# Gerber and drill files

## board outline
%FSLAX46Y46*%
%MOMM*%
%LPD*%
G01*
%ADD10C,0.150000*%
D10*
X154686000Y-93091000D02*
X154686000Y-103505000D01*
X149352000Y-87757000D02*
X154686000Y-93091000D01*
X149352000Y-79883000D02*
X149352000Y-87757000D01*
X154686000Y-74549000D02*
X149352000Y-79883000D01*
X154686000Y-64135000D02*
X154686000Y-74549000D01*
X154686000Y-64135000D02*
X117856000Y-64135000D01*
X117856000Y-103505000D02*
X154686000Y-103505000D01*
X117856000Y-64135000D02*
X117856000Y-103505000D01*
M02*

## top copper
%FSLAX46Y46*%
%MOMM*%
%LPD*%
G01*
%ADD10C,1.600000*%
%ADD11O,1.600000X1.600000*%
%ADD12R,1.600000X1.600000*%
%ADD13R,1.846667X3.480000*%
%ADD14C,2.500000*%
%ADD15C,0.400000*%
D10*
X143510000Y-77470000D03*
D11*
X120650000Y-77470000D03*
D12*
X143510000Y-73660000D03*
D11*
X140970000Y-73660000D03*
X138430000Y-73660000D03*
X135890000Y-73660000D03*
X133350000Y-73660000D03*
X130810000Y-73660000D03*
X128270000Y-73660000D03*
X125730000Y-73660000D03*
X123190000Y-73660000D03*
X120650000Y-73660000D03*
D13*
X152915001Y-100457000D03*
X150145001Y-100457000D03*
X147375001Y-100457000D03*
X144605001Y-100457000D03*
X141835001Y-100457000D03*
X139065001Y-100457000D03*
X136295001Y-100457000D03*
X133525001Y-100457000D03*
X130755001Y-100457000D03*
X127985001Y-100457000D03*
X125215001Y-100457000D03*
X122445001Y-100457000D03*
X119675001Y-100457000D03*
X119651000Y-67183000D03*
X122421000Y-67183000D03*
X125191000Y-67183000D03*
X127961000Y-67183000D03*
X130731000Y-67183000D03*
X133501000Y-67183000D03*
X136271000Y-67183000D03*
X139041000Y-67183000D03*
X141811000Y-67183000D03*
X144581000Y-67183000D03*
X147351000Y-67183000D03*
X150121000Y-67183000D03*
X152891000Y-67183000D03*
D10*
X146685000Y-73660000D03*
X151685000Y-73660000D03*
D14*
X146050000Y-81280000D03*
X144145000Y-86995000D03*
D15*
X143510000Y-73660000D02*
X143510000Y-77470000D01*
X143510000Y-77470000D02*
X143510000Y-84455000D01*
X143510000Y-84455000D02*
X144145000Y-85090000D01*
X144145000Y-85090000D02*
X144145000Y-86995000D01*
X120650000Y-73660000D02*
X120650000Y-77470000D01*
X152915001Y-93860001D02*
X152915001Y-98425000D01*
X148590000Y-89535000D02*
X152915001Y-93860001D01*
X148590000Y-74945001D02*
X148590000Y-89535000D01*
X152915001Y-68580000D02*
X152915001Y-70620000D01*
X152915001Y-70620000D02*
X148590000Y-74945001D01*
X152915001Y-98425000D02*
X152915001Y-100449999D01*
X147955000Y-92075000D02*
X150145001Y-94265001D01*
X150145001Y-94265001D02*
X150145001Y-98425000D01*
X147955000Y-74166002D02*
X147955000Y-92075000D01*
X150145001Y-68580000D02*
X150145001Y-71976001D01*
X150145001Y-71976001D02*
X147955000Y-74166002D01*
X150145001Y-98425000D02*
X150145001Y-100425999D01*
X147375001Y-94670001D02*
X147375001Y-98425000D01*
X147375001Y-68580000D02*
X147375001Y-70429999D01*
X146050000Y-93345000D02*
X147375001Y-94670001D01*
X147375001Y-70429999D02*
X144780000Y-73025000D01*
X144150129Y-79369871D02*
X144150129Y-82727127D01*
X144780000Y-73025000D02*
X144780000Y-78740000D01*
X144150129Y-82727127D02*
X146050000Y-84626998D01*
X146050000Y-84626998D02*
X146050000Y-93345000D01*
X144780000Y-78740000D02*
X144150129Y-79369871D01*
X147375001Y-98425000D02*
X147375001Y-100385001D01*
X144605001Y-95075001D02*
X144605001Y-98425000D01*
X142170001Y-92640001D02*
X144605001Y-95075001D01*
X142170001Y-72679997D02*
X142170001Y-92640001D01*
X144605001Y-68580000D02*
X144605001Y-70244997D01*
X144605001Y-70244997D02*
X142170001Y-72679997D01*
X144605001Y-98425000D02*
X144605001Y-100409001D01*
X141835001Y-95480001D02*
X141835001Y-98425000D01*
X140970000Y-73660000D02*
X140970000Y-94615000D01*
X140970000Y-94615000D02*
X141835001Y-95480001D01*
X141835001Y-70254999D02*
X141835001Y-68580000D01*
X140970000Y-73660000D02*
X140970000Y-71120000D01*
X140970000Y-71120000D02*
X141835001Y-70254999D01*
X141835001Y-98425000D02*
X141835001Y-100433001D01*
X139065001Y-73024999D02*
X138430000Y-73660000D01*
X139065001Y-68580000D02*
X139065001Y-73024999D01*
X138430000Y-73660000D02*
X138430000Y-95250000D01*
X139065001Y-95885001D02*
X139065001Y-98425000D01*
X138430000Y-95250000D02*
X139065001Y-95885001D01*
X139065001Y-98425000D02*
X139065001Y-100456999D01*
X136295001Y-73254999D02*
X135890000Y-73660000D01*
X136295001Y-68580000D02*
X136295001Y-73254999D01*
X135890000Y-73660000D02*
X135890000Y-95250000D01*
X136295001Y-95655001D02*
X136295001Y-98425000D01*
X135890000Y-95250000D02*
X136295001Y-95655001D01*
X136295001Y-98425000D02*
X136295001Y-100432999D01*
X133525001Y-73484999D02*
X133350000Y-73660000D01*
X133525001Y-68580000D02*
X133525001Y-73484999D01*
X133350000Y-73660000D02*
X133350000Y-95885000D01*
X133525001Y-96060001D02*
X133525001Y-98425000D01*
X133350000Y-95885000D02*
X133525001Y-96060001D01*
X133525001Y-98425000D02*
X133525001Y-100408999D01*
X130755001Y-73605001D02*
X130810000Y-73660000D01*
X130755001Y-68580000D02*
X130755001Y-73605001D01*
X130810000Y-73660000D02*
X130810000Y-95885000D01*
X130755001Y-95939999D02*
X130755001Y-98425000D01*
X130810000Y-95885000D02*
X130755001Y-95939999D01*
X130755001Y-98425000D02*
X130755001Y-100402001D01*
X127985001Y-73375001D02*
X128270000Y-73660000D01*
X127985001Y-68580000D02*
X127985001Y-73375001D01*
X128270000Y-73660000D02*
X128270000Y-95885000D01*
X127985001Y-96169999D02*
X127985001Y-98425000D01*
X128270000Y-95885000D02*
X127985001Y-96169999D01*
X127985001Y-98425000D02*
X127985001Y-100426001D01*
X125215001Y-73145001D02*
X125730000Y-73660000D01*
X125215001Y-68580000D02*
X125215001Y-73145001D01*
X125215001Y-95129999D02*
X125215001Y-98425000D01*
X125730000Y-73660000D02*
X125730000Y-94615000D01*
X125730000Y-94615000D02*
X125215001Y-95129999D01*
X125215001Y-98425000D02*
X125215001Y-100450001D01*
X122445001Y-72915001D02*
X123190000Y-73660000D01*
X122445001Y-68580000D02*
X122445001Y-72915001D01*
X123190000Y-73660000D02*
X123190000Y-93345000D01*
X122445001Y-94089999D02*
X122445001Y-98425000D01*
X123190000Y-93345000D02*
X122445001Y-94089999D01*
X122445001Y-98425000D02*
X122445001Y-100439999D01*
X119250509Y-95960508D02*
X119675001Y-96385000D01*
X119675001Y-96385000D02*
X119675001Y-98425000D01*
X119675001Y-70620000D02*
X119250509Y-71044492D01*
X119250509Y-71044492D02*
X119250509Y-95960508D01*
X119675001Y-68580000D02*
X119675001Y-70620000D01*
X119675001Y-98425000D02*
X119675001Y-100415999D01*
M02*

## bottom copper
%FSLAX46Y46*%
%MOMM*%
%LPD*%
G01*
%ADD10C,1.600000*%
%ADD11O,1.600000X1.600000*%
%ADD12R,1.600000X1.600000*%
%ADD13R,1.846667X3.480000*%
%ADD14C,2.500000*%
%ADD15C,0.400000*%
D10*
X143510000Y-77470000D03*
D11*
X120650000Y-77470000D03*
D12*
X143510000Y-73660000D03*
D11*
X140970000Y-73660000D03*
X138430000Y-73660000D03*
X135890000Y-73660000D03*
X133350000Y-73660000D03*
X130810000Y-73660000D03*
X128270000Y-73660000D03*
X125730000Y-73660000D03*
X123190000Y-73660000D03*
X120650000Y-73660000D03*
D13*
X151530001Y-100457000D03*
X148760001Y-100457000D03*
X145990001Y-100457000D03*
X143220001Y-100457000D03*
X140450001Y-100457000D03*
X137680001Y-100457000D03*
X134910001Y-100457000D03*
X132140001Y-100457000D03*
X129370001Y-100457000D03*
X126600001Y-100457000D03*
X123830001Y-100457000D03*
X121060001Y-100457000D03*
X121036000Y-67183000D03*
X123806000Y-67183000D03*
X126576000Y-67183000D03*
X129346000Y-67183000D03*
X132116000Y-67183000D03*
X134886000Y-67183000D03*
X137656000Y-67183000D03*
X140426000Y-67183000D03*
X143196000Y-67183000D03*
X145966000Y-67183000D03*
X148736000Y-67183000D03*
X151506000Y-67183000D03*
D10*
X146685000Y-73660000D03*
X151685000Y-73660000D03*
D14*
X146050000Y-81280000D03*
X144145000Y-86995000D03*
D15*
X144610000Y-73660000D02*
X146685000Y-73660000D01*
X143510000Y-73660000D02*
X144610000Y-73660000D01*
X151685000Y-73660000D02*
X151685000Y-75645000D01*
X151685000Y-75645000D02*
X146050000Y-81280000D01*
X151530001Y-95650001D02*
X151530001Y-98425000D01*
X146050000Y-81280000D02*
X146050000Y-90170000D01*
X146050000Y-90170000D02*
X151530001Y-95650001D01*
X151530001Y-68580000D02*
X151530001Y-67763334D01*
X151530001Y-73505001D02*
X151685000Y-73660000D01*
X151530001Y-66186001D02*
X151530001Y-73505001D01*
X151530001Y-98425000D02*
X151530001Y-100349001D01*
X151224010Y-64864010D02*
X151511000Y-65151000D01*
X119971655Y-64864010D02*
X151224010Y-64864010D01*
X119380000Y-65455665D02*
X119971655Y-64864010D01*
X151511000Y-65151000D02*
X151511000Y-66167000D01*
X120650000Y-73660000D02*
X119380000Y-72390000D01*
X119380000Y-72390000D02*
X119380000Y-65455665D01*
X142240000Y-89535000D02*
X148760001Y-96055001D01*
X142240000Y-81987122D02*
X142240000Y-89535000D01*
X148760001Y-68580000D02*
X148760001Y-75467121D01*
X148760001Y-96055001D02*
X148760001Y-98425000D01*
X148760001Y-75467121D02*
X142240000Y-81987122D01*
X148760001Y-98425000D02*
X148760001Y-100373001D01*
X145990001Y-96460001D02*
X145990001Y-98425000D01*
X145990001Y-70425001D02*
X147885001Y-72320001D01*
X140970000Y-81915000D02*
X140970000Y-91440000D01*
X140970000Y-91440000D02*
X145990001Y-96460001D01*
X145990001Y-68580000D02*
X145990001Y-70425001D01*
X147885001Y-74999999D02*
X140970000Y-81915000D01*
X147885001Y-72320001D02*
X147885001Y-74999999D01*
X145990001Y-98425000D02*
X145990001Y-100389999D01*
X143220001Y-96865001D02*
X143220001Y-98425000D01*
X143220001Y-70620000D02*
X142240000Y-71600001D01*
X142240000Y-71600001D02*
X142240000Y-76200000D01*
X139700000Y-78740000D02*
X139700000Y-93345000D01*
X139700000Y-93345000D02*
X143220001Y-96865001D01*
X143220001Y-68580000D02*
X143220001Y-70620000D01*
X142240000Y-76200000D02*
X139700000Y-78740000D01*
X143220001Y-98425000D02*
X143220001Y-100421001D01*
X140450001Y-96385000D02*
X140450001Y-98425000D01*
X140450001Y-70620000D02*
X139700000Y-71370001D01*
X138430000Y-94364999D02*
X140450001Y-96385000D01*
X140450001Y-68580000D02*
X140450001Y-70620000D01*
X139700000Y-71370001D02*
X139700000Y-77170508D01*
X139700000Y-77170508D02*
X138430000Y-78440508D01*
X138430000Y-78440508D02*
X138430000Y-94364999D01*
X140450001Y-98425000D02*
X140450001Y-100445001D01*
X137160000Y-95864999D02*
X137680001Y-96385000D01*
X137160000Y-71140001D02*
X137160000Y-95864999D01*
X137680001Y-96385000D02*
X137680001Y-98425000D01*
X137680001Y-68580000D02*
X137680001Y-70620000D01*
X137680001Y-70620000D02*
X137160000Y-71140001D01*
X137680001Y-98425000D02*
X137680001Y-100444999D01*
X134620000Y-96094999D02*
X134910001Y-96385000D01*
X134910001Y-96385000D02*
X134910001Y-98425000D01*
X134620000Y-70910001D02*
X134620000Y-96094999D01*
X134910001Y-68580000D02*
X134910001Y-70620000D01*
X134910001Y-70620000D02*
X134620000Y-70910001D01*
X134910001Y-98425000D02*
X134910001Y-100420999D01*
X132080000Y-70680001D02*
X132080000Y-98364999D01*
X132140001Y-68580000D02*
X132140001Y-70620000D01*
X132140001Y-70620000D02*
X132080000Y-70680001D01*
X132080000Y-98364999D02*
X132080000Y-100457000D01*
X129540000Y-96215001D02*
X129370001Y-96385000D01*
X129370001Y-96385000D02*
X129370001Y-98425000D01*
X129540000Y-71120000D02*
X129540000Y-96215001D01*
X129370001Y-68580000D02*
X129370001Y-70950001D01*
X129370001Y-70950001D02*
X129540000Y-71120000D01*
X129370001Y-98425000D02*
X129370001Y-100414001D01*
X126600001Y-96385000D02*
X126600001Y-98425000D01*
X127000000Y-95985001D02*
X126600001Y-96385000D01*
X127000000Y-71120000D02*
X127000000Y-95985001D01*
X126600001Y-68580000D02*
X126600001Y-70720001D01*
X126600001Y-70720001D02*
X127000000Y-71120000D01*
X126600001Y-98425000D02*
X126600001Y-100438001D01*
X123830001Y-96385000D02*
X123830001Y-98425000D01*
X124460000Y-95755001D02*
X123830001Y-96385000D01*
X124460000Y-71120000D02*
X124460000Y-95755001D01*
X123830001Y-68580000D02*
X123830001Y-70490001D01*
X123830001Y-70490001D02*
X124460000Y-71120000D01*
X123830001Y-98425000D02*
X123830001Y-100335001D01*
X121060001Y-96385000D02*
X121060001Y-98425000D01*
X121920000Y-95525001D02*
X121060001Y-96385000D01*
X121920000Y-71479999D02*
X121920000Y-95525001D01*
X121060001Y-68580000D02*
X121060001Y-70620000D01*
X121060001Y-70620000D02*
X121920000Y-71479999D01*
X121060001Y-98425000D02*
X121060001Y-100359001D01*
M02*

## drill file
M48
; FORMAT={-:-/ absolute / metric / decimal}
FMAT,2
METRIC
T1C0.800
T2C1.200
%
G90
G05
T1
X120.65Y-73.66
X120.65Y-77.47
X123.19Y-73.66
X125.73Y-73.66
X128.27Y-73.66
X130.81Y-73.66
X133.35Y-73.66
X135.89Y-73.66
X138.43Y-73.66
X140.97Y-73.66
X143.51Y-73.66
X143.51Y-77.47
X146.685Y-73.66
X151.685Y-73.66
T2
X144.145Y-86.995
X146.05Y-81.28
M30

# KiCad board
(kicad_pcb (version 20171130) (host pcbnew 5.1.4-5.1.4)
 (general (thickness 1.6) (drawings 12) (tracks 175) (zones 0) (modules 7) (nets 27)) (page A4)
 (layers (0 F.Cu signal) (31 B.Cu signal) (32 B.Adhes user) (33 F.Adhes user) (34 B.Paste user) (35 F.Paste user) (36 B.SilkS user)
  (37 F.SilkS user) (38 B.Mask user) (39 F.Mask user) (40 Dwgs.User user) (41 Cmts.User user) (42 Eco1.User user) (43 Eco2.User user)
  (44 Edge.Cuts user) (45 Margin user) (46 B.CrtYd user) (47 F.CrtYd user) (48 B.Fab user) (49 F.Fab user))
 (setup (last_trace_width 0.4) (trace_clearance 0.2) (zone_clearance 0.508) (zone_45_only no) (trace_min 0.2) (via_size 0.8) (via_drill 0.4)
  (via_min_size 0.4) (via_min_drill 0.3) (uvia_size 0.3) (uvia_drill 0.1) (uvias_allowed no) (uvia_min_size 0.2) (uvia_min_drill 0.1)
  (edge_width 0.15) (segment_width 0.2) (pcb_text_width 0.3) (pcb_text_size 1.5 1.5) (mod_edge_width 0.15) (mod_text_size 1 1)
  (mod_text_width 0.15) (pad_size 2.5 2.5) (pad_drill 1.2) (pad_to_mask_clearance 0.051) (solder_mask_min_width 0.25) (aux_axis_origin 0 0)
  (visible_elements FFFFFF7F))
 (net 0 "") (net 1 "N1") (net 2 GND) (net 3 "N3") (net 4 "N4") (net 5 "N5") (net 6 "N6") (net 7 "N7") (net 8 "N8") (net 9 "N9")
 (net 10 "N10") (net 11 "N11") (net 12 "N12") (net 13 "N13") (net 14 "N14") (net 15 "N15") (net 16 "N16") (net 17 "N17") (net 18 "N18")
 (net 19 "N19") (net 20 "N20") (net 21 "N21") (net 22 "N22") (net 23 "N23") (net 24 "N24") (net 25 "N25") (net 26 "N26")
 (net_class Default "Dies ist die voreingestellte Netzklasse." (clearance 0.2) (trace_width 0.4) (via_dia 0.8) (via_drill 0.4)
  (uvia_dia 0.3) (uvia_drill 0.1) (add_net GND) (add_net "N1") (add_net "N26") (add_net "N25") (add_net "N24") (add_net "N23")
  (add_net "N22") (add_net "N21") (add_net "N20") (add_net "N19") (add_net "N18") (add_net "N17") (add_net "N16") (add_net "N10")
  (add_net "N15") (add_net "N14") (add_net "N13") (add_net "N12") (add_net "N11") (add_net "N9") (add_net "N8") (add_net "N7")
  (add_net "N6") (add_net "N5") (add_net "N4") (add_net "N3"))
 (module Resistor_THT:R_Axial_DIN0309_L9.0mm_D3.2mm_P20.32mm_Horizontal (layer B.Cu) (at 143.51 77.47 180)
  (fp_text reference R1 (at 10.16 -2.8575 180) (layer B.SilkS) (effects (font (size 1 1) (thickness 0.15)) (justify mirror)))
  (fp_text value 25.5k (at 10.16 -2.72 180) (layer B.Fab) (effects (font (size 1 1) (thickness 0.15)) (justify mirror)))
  (pad 1 thru_hole circle (at 0 0 180) (size 1.6 1.6) (drill 0.8) (layers *.Cu *.Mask) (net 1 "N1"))
  (pad 2 thru_hole oval (at 22.86 0 180) (size 1.6 1.6) (drill 0.8) (layers *.Cu *.Mask) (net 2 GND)))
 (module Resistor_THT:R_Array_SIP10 (layer B.Cu) (at 143.51 73.66 180)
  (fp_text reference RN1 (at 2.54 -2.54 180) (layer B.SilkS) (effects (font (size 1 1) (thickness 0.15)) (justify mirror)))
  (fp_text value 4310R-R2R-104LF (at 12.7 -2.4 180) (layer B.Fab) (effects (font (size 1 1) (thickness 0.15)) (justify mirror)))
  (pad 1 thru_hole rect (at 0 0 180) (size 1.6 1.6) (drill 0.8) (layers *.Cu *.Mask) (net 1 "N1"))
  (pad 2 thru_hole oval (at 2.54 0 180) (size 1.6 1.6) (drill 0.8) (layers *.Cu *.Mask) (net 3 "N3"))
  (pad 3 thru_hole oval (at 5.08 0 180) (size 1.6 1.6) (drill 0.8) (layers *.Cu *.Mask) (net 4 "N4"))
  (pad 4 thru_hole oval (at 7.62 0 180) (size 1.6 1.6) (drill 0.8) (layers *.Cu *.Mask) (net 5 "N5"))
  (pad 5 thru_hole oval (at 10.16 0 180) (size 1.6 1.6) (drill 0.8) (layers *.Cu *.Mask) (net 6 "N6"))
  (pad 6 thru_hole oval (at 12.7 0 180) (size 1.6 1.6) (drill 0.8) (layers *.Cu *.Mask) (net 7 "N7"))
  (pad 7 thru_hole oval (at 15.24 0 180) (size 1.6 1.6) (drill 0.8) (layers *.Cu *.Mask) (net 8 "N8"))
  (pad 8 thru_hole oval (at 17.78 0 180) (size 1.6 1.6) (drill 0.8) (layers *.Cu *.Mask) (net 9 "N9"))
  (pad 9 thru_hole oval (at 20.32 0 180) (size 1.6 1.6) (drill 0.8) (layers *.Cu *.Mask) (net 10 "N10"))
  (pad 10 thru_hole oval (at 22.86 0 180) (size 1.6 1.6) (drill 0.8) (layers *.Cu *.Mask) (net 2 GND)))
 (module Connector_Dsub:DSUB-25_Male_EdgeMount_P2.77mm (layer F.Cu) (at 136.295001 100.457)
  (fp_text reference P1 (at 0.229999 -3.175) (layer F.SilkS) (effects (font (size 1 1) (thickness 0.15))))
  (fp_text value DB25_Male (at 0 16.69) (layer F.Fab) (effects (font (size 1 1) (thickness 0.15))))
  (pad 25 smd rect (at 15.235 0) (size 1.846667 3.48) (layers B.Cu B.Paste B.Mask) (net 2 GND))
  (pad 24 smd rect (at 12.465 0) (size 1.846667 3.48) (layers B.Cu B.Paste B.Mask) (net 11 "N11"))
  (pad 23 smd rect (at 9.695 0) (size 1.846667 3.48) (layers B.Cu B.Paste B.Mask) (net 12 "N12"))
  (pad 22 smd rect (at 6.925 0) (size 1.846667 3.48) (layers B.Cu B.Paste B.Mask) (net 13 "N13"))
  (pad 21 smd rect (at 4.155 0) (size 1.846667 3.48) (layers B.Cu B.Paste B.Mask) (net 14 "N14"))
  (pad 20 smd rect (at 1.385 0) (size 1.846667 3.48) (layers B.Cu B.Paste B.Mask) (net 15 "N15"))
  (pad 19 smd rect (at -1.385 0) (size 1.846667 3.48) (layers B.Cu B.Paste B.Mask) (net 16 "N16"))
  (pad 18 smd rect (at -4.155 0) (size 1.846667 3.48) (layers B.Cu B.Paste B.Mask) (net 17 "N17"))
  (pad 17 smd rect (at -6.925 0) (size 1.846667 3.48) (layers B.Cu B.Paste B.Mask) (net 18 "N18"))
  (pad 16 smd rect (at -9.695 0) (size 1.846667 3.48) (layers B.Cu B.Paste B.Mask) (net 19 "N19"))
  (pad 15 smd rect (at -12.465 0) (size 1.846667 3.48) (layers B.Cu B.Paste B.Mask) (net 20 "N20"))
  (pad 14 smd rect (at -15.235 0) (size 1.846667 3.48) (layers B.Cu B.Paste B.Mask) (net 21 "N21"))
  (pad 13 smd rect (at 16.62 0) (size 1.846667 3.48) (layers F.Cu F.Paste F.Mask) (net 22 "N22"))
  (pad 12 smd rect (at 13.85 0) (size 1.846667 3.48) (layers F.Cu F.Paste F.Mask) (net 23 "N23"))
  (pad 11 smd rect (at 11.08 0) (size 1.846667 3.48) (layers F.Cu F.Paste F.Mask) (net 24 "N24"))
  (pad 10 smd rect (at 8.31 0) (size 1.846667 3.48) (layers F.Cu F.Paste F.Mask) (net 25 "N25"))
  (pad 9 smd rect (at 5.54 0) (size 1.846667 3.48) (layers F.Cu F.Paste F.Mask) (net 3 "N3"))
  (pad 8 smd rect (at 2.77 0) (size 1.846667 3.48) (layers F.Cu F.Paste F.Mask) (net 4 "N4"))
  (pad 7 smd rect (at 0 0) (size 1.846667 3.48) (layers F.Cu F.Paste F.Mask) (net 5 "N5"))
  (pad 6 smd rect (at -2.77 0) (size 1.846667 3.48) (layers F.Cu F.Paste F.Mask) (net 6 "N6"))
  (pad 5 smd rect (at -5.54 0) (size 1.846667 3.48) (layers F.Cu F.Paste F.Mask) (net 7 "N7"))
  (pad 4 smd rect (at -8.31 0) (size 1.846667 3.48) (layers F.Cu F.Paste F.Mask) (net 8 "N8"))
  (pad 3 smd rect (at -11.08 0) (size 1.846667 3.48) (layers F.Cu F.Paste F.Mask) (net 9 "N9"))
  (pad 2 smd rect (at -13.85 0) (size 1.846667 3.48) (layers F.Cu F.Paste F.Mask) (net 10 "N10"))
  (pad 1 smd rect (at -16.62 0) (size 1.846667 3.48) (layers F.Cu F.Paste F.Mask) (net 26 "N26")))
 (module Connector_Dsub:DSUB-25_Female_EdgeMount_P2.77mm (layer F.Cu) (at 136.271 67.183 180)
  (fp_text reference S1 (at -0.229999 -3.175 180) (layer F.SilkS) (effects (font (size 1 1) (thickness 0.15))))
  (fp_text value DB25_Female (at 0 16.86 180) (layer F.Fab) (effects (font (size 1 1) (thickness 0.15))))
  (pad 1 smd rect (at 16.62 0 180) (size 1.846667 3.48) (layers F.Cu F.Paste F.Mask) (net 26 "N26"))
  (pad 2 smd rect (at 13.85 0 180) (size 1.846667 3.48) (layers F.Cu F.Paste F.Mask) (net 10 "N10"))
  (pad 3 smd rect (at 11.08 0 180) (size 1.846667 3.48) (layers F.Cu F.Paste F.Mask) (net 9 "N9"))
  (pad 4 smd rect (at 8.31 0 180) (size 1.846667 3.48) (layers F.Cu F.Paste F.Mask) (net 8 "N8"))
  (pad 5 smd rect (at 5.54 0 180) (size 1.846667 3.48) (layers F.Cu F.Paste F.Mask) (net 7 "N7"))
  (pad 6 smd rect (at 2.77 0 180) (size 1.846667 3.48) (layers F.Cu F.Paste F.Mask) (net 6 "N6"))
  (pad 7 smd rect (at 0 0 180) (size 1.846667 3.48) (layers F.Cu F.Paste F.Mask) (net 5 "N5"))
  (pad 8 smd rect (at -2.77 0 180) (size 1.846667 3.48) (layers F.Cu F.Paste F.Mask) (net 4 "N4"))
  (pad 9 smd rect (at -5.54 0 180) (size 1.846667 3.48) (layers F.Cu F.Paste F.Mask) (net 3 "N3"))
  (pad 10 smd rect (at -8.31 0 180) (size 1.846667 3.48) (layers F.Cu F.Paste F.Mask) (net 25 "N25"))
  (pad 11 smd rect (at -11.08 0 180) (size 1.846667 3.48) (layers F.Cu F.Paste F.Mask) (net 24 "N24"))
  (pad 12 smd rect (at -13.85 0 180) (size 1.846667 3.48) (layers F.Cu F.Paste F.Mask) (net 23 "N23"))
  (pad 13 smd rect (at -16.62 0 180) (size 1.846667 3.48) (layers F.Cu F.Paste F.Mask) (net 22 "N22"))
  (pad 14 smd rect (at 15.235 0 180) (size 1.846667 3.48) (layers B.Cu B.Paste B.Mask) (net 21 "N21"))
  (pad 15 smd rect (at 12.465 0 180) (size 1.846667 3.48) (layers B.Cu B.Paste B.Mask) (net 20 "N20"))
  (pad 16 smd rect (at 9.695 0 180) (size 1.846667 3.48) (layers B.Cu B.Paste B.Mask) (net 19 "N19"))
  (pad 17 smd rect (at 6.925 0 180) (size 1.846667 3.48) (layers B.Cu B.Paste B.Mask) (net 18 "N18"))
  (pad 18 smd rect (at 4.155 0 180) (size 1.846667 3.48) (layers B.Cu B.Paste B.Mask) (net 17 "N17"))
  (pad 19 smd rect (at 1.385 0 180) (size 1.846667 3.48) (layers B.Cu B.Paste B.Mask) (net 16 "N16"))
  (pad 20 smd rect (at -1.385 0 180) (size 1.846667 3.48) (layers B.Cu B.Paste B.Mask) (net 15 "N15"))
  (pad 21 smd rect (at -4.155 0 180) (size 1.846667 3.48) (layers B.Cu B.Paste B.Mask) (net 14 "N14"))
  (pad 22 smd rect (at -6.925 0 180) (size 1.846667 3.48) (layers B.Cu B.Paste B.Mask) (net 13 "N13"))
  (pad 23 smd rect (at -9.695 0 180) (size 1.846667 3.48) (layers B.Cu B.Paste B.Mask) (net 12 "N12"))
  (pad 24 smd rect (at -12.465 0 180) (size 1.846667 3.48) (layers B.Cu B.Paste B.Mask) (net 11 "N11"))
  (pad 25 smd rect (at -15.235 0 180) (size 1.846667 3.48) (layers B.Cu B.Paste B.Mask) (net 2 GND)))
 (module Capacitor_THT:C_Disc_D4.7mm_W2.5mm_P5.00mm (layer B.Cu) (at 146.685 73.66)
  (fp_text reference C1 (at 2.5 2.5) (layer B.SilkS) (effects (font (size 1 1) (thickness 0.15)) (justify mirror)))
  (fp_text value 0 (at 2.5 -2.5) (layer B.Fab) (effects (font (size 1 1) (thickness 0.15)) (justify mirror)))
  (pad 1 thru_hole circle (at 0 0) (size 1.6 1.6) (drill 0.8) (layers *.Cu *.Mask) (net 1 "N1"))
  (pad 2 thru_hole circle (at 5 0) (size 1.6 1.6) (drill 0.8) (layers *.Cu *.Mask) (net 2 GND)))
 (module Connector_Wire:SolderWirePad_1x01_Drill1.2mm (layer F.Cu) (at 146.05 81.28)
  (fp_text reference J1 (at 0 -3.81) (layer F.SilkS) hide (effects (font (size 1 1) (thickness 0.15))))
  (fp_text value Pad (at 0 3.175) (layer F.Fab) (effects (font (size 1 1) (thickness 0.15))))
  (pad 1 thru_hole circle (at 0 0) (size 2.5 2.5) (drill 1.2) (layers *.Cu *.Mask) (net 2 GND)))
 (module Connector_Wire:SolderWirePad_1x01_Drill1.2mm (layer F.Cu) (at 144.145 86.995)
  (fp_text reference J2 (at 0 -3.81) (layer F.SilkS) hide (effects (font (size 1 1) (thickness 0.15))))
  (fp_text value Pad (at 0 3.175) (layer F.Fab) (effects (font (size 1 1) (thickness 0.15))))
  (pad 1 thru_hole circle (at 0 0) (size 2.5 2.5) (drill 1.2) (layers *.Cu *.Mask) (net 1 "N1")))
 (gr_line (start 154.686 93.091) (end 154.686 103.505) (layer Edge.Cuts) (width 0.15))
 (gr_line (start 149.352 87.757) (end 154.686 93.091) (layer Edge.Cuts) (width 0.15))
 (gr_line (start 149.352 79.883) (end 149.352 87.757) (layer Edge.Cuts) (width 0.15))
 (gr_line (start 154.686 74.549) (end 149.352 79.883) (layer Edge.Cuts) (width 0.15))
 (gr_line (start 154.686 64.135) (end 154.686 74.549) (layer Edge.Cuts) (width 0.15))
 (gr_line (start 154.686 64.135) (end 117.856 64.135) (layer Edge.Cuts) (width 0.15))
 (gr_line (start 117.856 103.505) (end 154.686 103.505) (layer Edge.Cuts) (width 0.15))
 (gr_line (start 117.856 64.135) (end 117.856 103.505) (layer Edge.Cuts) (width 0.15))
 (segment (start 144.61 73.66) (end 146.685 73.66) (width 0.4) (layer B.Cu) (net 1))
 (segment (start 143.51 73.66) (end 144.61 73.66) (width 0.4) (layer B.Cu) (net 1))
 (segment (start 143.51 73.66) (end 143.51 77.47) (width 0.4) (layer F.Cu) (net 1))
 (segment (start 143.51 77.47) (end 143.51 84.455) (width 0.4) (layer F.Cu) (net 1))
 (segment (start 143.51 84.455) (end 144.145 85.09) (width 0.4) (layer F.Cu) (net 1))
 (segment (start 144.145 85.09) (end 144.145 86.995) (width 0.4) (layer F.Cu) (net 1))
 (segment (start 120.65 73.66) (end 120.65 77.47) (width 0.4) (layer F.Cu) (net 2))
 (segment (start 151.685 73.66) (end 151.685 75.645) (width 0.4) (layer B.Cu) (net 2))
 (segment (start 151.685 75.645) (end 146.05 81.28) (width 0.4) (layer B.Cu) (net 2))
 (segment (start 151.530001 95.650001) (end 151.530001 98.425) (width 0.4) (layer B.Cu) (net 2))
 (segment (start 146.05 81.28) (end 146.05 90.17) (width 0.4) (layer B.Cu) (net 2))
 (segment (start 146.05 90.17) (end 151.530001 95.650001) (width 0.4) (layer B.Cu) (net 2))
 (segment (start 151.530001 68.58) (end 151.530001 67.763334) (width 0.4) (layer B.Cu) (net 2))
 (segment (start 151.530001 73.505001) (end 151.685 73.66) (width 0.4) (layer B.Cu) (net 2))
 (segment (start 151.530001 66.186001) (end 151.530001 73.505001) (width 0.4) (layer B.Cu) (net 2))
 (segment (start 151.530001 98.425) (end 151.530001 100.349001) (width 0.4) (layer B.Cu) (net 2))
 (segment (start 151.22401 64.86401) (end 151.511 65.151) (width 0.4) (layer B.Cu) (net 2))
 (segment (start 119.971655 64.86401) (end 151.22401 64.86401) (width 0.4) (layer B.Cu) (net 2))
 (segment (start 119.38 65.455665) (end 119.971655 64.86401) (width 0.4) (layer B.Cu) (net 2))
 (segment (start 151.511 65.151) (end 151.511 66.167) (width 0.4) (layer B.Cu) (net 2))
 (segment (start 120.65 73.66) (end 119.38 72.39) (width 0.4) (layer B.Cu) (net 2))
 (segment (start 119.38 72.39) (end 119.38 65.455665) (width 0.4) (layer B.Cu) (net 2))
 (segment (start 142.24 89.535) (end 148.760001 96.055001) (width 0.4) (layer B.Cu) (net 11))
 (segment (start 142.24 81.987122) (end 142.24 89.535) (width 0.4) (layer B.Cu) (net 11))
 (segment (start 148.760001 68.58) (end 148.760001 75.467121) (width 0.4) (layer B.Cu) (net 11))
 (segment (start 148.760001 96.055001) (end 148.760001 98.425) (width 0.4) (layer B.Cu) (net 11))
 (segment (start 148.760001 75.467121) (end 142.24 81.987122) (width 0.4) (layer B.Cu) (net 11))
 (segment (start 148.760001 98.425) (end 148.760001 100.373001) (width 0.4) (layer B.Cu) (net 11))
 (segment (start 145.990001 96.460001) (end 145.990001 98.425) (width 0.4) (layer B.Cu) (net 12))
 (segment (start 145.990001 70.425001) (end 147.885001 72.320001) (width 0.4) (layer B.Cu) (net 12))
 (segment (start 140.97 81.915) (end 140.97 91.44) (width 0.4) (layer B.Cu) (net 12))
 (segment (start 140.97 91.44) (end 145.990001 96.460001) (width 0.4) (layer B.Cu) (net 12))
 (segment (start 145.990001 68.58) (end 145.990001 70.425001) (width 0.4) (layer B.Cu) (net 12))
 (segment (start 147.885001 74.999999) (end 140.97 81.915) (width 0.4) (layer B.Cu) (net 12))
 (segment (start 147.885001 72.320001) (end 147.885001 74.999999) (width 0.4) (layer B.Cu) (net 12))
 (segment (start 145.990001 98.425) (end 145.990001 100.389999) (width 0.4) (layer B.Cu) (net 12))
 (segment (start 143.220001 96.865001) (end 143.220001 98.425) (width 0.4) (layer B.Cu) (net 13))
 (segment (start 143.220001 70.62) (end 142.24 71.600001) (width 0.4) (layer B.Cu) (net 13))
 (segment (start 142.24 71.600001) (end 142.24 76.2) (width 0.4) (layer B.Cu) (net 13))
 (segment (start 139.7 78.74) (end 139.7 93.345) (width 0.4) (layer B.Cu) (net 13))
 (segment (start 139.7 93.345) (end 143.220001 96.865001) (width 0.4) (layer B.Cu) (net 13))
 (segment (start 143.220001 68.58) (end 143.220001 70.62) (width 0.4) (layer B.Cu) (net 13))
 (segment (start 142.24 76.2) (end 139.7 78.74) (width 0.4) (layer B.Cu) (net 13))
 (segment (start 143.220001 98.425) (end 143.220001 100.421001) (width 0.4) (layer B.Cu) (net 13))
 (segment (start 140.450001 96.385) (end 140.450001 98.425) (width 0.4) (layer B.Cu) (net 14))
 (segment (start 140.450001 70.62) (end 139.7 71.370001) (width 0.4) (layer B.Cu) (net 14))
 (segment (start 138.43 94.364999) (end 140.450001 96.385) (width 0.4) (layer B.Cu) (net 14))
 (segment (start 140.450001 68.58) (end 140.450001 70.62) (width 0.4) (layer B.Cu) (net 14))
 (segment (start 139.7 71.370001) (end 139.7 77.170508) (width 0.4) (layer B.Cu) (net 14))
 (segment (start 139.7 77.170508) (end 138.43 78.440508) (width 0.4) (layer B.Cu) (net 14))
 (segment (start 138.43 78.440508) (end 138.43 94.364999) (width 0.4) (layer B.Cu) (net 14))
 (segment (start 140.450001 98.425) (end 140.450001 100.445001) (width 0.4) (layer B.Cu) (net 14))
 (segment (start 137.16 95.864999) (end 137.680001 96.385) (width 0.4) (layer B.Cu) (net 15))
 (segment (start 137.16 71.140001) (end 137.16 95.864999) (width 0.4) (layer B.Cu) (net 15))
 (segment (start 137.680001 96.385) (end 137.680001 98.425) (width 0.4) (layer B.Cu) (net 15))
 (segment (start 137.680001 68.58) (end 137.680001 70.62) (width 0.4) (layer B.Cu) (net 15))
 (segment (start 137.680001 70.62) (end 137.16 71.140001) (width 0.4) (layer B.Cu) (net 15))
 (segment (start 137.680001 98.425) (end 137.680001 100.444999) (width 0.4) (layer B.Cu) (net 15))
 (segment (start 134.62 96.094999) (end 134.910001 96.385) (width 0.4) (layer B.Cu) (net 16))
 (segment (start 134.910001 96.385) (end 134.910001 98.425) (width 0.4) (layer B.Cu) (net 16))
 (segment (start 134.62 70.910001) (end 134.62 96.094999) (width 0.4) (layer B.Cu) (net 16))
 (segment (start 134.910001 68.58) (end 134.910001 70.62) (width 0.4) (layer B.Cu) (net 16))
 (segment (start 134.910001 70.62) (end 134.62 70.910001) (width 0.4) (layer B.Cu) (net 16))
 (segment (start 134.910001 98.425) (end 134.910001 100.420999) (width 0.4) (layer B.Cu) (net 16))
 (segment (start 132.08 70.680001) (end 132.08 98.364999) (width 0.4) (layer B.Cu) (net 17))
 (segment (start 132.140001 68.58) (end 132.140001 70.62) (width 0.4) (layer B.Cu) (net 17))
 (segment (start 132.140001 70.62) (end 132.08 70.680001) (width 0.4) (layer B.Cu) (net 17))
 (segment (start 132.08 98.364999) (end 132.08 100.457) (width 0.4) (layer B.Cu) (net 17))
 (segment (start 129.54 96.215001) (end 129.370001 96.385) (width 0.4) (layer B.Cu) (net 18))
 (segment (start 129.370001 96.385) (end 129.370001 98.425) (width 0.4) (layer B.Cu) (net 18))
 (segment (start 129.54 71.12) (end 129.54 96.215001) (width 0.4) (layer B.Cu) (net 18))
 (segment (start 129.370001 68.58) (end 129.370001 70.950001) (width 0.4) (layer B.Cu) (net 18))
 (segment (start 129.370001 70.950001) (end 129.54 71.12) (width 0.4) (layer B.Cu) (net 18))
 (segment (start 129.370001 98.425) (end 129.370001 100.414001) (width 0.4) (layer B.Cu) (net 18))
 (segment (start 126.600001 96.385) (end 126.600001 98.425) (width 0.4) (layer B.Cu) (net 19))
 (segment (start 127 95.985001) (end 126.600001 96.385) (width 0.4) (layer B.Cu) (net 19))
 (segment (start 127 71.12) (end 127 95.985001) (width 0.4) (layer B.Cu) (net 19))
 (segment (start 126.600001 68.58) (end 126.600001 70.720001) (width 0.4) (layer B.Cu) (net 19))
 (segment (start 126.600001 70.720001) (end 127 71.12) (width 0.4) (layer B.Cu) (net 19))
 (segment (start 126.600001 98.425) (end 126.600001 100.438001) (width 0.4) (layer B.Cu) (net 19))
 (segment (start 123.830001 96.385) (end 123.830001 98.425) (width 0.4) (layer B.Cu) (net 20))
 (segment (start 124.46 95.755001) (end 123.830001 96.385) (width 0.4) (layer B.Cu) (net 20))
 (segment (start 124.46 71.12) (end 124.46 95.755001) (width 0.4) (layer B.Cu) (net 20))
 (segment (start 123.830001 68.58) (end 123.830001 70.490001) (width 0.4) (layer B.Cu) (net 20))
 (segment (start 123.830001 70.490001) (end 124.46 71.12) (width 0.4) (layer B.Cu) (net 20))
 (segment (start 123.830001 98.425) (end 123.830001 100.335001) (width 0.4) (layer B.Cu) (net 20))
 (segment (start 121.060001 96.385) (end 121.060001 98.425) (width 0.4) (layer B.Cu) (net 21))
 (segment (start 121.92 95.525001) (end 121.060001 96.385) (width 0.4) (layer B.Cu) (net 21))
 (segment (start 121.92 71.479999) (end 121.92 95.525001) (width 0.4) (layer B.Cu) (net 21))
 (segment (start 121.060001 68.58) (end 121.060001 70.62) (width 0.4) (layer B.Cu) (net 21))
 (segment (start 121.060001 70.62) (end 121.92 71.479999) (width 0.4) (layer B.Cu) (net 21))
 (segment (start 121.060001 98.425) (end 121.060001 100.359001) (width 0.4) (layer B.Cu) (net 21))
 (segment (start 152.915001 93.860001) (end 152.915001 98.425) (width 0.4) (layer F.Cu) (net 22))
 (segment (start 148.59 89.535) (end 152.915001 93.860001) (width 0.4) (layer F.Cu) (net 22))
 (segment (start 148.59 74.945001) (end 148.59 89.535) (width 0.4) (layer F.Cu) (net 22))
 (segment (start 152.915001 68.58) (end 152.915001 70.62) (width 0.4) (layer F.Cu) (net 22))
 (segment (start 152.915001 70.62) (end 148.59 74.945001) (width 0.4) (layer F.Cu) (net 22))
 (segment (start 152.915001 98.425) (end 152.915001 100.449999) (width 0.4) (layer F.Cu) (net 22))
 (segment (start 147.955 92.075) (end 150.145001 94.265001) (width 0.4) (layer F.Cu) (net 23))
 (segment (start 150.145001 94.265001) (end 150.145001 98.425) (width 0.4) (layer F.Cu) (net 23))
 (segment (start 147.955 74.166002) (end 147.955 92.075) (width 0.4) (layer F.Cu) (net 23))
 (segment (start 150.145001 68.58) (end 150.145001 71.976001) (width 0.4) (layer F.Cu) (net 23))
 (segment (start 150.145001 71.976001) (end 147.955 74.166002) (width 0.4) (layer F.Cu) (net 23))
 (segment (start 150.145001 98.425) (end 150.145001 100.425999) (width 0.4) (layer F.Cu) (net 23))
 (segment (start 147.375001 94.670001) (end 147.375001 98.425) (width 0.4) (layer F.Cu) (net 24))
 (segment (start 147.375001 68.58) (end 147.375001 70.429999) (width 0.4) (layer F.Cu) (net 24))
 (segment (start 146.05 93.345) (end 147.375001 94.670001) (width 0.4) (layer F.Cu) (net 24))
 (segment (start 147.375001 70.429999) (end 144.78 73.025) (width 0.4) (layer F.Cu) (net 24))
 (segment (start 144.150129 79.369871) (end 144.150129 82.727127) (width 0.4) (layer F.Cu) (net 24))
 (segment (start 144.78 73.025) (end 144.78 78.74) (width 0.4) (layer F.Cu) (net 24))
 (segment (start 144.150129 82.727127) (end 146.05 84.626998) (width 0.4) (layer F.Cu) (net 24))
 (segment (start 146.05 84.626998) (end 146.05 93.345) (width 0.4) (layer F.Cu) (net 24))
 (segment (start 144.78 78.74) (end 144.150129 79.369871) (width 0.4) (layer F.Cu) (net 24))
 (segment (start 147.375001 98.425) (end 147.375001 100.385001) (width 0.4) (layer F.Cu) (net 24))
 (segment (start 144.605001 95.075001) (end 144.605001 98.425) (width 0.4) (layer F.Cu) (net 25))
 (segment (start 142.170001 92.640001) (end 144.605001 95.075001) (width 0.4) (layer F.Cu) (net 25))
 (segment (start 142.170001 72.679997) (end 142.170001 92.640001) (width 0.4) (layer F.Cu) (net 25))
 (segment (start 144.605001 68.58) (end 144.605001 70.244997) (width 0.4) (layer F.Cu) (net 25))
 (segment (start 144.605001 70.244997) (end 142.170001 72.679997) (width 0.4) (layer F.Cu) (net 25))
 (segment (start 144.605001 98.425) (end 144.605001 100.409001) (width 0.4) (layer F.Cu) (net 25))
 (segment (start 141.835001 95.480001) (end 141.835001 98.425) (width 0.4) (layer F.Cu) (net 3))
 (segment (start 140.97 73.66) (end 140.97 94.615) (width 0.4) (layer F.Cu) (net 3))
 (segment (start 140.97 94.615) (end 141.835001 95.480001) (width 0.4) (layer F.Cu) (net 3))
 (segment (start 141.835001 70.254999) (end 141.835001 68.58) (width 0.4) (layer F.Cu) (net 3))
 (segment (start 140.97 73.66) (end 140.97 71.12) (width 0.4) (layer F.Cu) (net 3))
 (segment (start 140.97 71.12) (end 141.835001 70.254999) (width 0.4) (layer F.Cu) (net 3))
 (segment (start 141.835001 98.425) (end 141.835001 100.433001) (width 0.4) (layer F.Cu) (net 3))
 (segment (start 139.065001 73.024999) (end 138.43 73.66) (width 0.4) (layer F.Cu) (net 4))
 (segment (start 139.065001 68.58) (end 139.065001 73.024999) (width 0.4) (layer F.Cu) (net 4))
 (segment (start 138.43 73.66) (end 138.43 95.25) (width 0.4) (layer F.Cu) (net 4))
 (segment (start 139.065001 95.885001) (end 139.065001 98.425) (width 0.4) (layer F.Cu) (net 4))
 (segment (start 138.43 95.25) (end 139.065001 95.885001) (width 0.4) (layer F.Cu) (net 4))
 (segment (start 139.065001 98.425) (end 139.065001 100.456999) (width 0.4) (layer F.Cu) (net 4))
 (segment (start 136.295001 73.254999) (end 135.89 73.66) (width 0.4) (layer F.Cu) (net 5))
 (segment (start 136.295001 68.58) (end 136.295001 73.254999) (width 0.4) (layer F.Cu) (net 5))
 (segment (start 135.89 73.66) (end 135.89 95.25) (width 0.4) (layer F.Cu) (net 5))
 (segment (start 136.295001 95.655001) (end 136.295001 98.425) (width 0.4) (layer F.Cu) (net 5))
 (segment (start 135.89 95.25) (end 136.295001 95.655001) (width 0.4) (layer F.Cu) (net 5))
 (segment (start 136.295001 98.425) (end 136.295001 100.432999) (width 0.4) (layer F.Cu) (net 5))
 (segment (start 133.525001 73.484999) (end 133.35 73.66) (width 0.4) (layer F.Cu) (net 6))
 (segment (start 133.525001 68.58) (end 133.525001 73.484999) (width 0.4) (layer F.Cu) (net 6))
 (segment (start 133.35 73.66) (end 133.35 95.885) (width 0.4) (layer F.Cu) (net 6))
 (segment (start 133.525001 96.060001) (end 133.525001 98.425) (width 0.4) (layer F.Cu) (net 6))
 (segment (start 133.35 95.885) (end 133.525001 96.060001) (width 0.4) (layer F.Cu) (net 6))
 (segment (start 133.525001 98.425) (end 133.525001 100.408999) (width 0.4) (layer F.Cu) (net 6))
 (segment (start 130.755001 73.605001) (end 130.81 73.66) (width 0.4) (layer F.Cu) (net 7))
 (segment (start 130.755001 68.58) (end 130.755001 73.605001) (width 0.4) (layer F.Cu) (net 7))
 (segment (start 130.81 73.66) (end 130.81 95.885) (width 0.4) (layer F.Cu) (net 7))
 (segment (start 130.755001 95.939999) (end 130.755001 98.425) (width 0.4) (layer F.Cu) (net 7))
 (segment (start 130.81 95.885) (end 130.755001 95.939999) (width 0.4) (layer F.Cu) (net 7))
 (segment (start 130.755001 98.425) (end 130.755001 100.402001) (width 0.4) (layer F.Cu) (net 7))
 (segment (start 127.985001 73.375001) (end 128.27 73.66) (width 0.4) (layer F.Cu) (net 8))
 (segment (start 127.985001 68.58) (end 127.985001 73.375001) (width 0.4) (layer F.Cu) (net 8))
 (segment (start 128.27 73.66) (end 128.27 95.885) (width 0.4) (layer F.Cu) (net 8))
 (segment (start 127.985001 96.169999) (end 127.985001 98.425) (width 0.4) (layer F.Cu) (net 8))
 (segment (start 128.27 95.885) (end 127.985001 96.169999) (width 0.4) (layer F.Cu) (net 8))
 (segment (start 127.985001 98.425) (end 127.985001 100.426001) (width 0.4) (layer F.Cu) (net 8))
 (segment (start 125.215001 73.145001) (end 125.73 73.66) (width 0.4) (layer F.Cu) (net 9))
 (segment (start 125.215001 68.58) (end 125.215001 73.145001) (width 0.4) (layer F.Cu) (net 9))
 (segment (start 125.215001 95.129999) (end 125.215001 98.425) (width 0.4) (layer F.Cu) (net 9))
 (segment (start 125.73 73.66) (end 125.73 94.615) (width 0.4) (layer F.Cu) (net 9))
 (segment (start 125.73 94.615) (end 125.215001 95.129999) (width 0.4) (layer F.Cu) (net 9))
 (segment (start 125.215001 98.425) (end 125.215001 100.450001) (width 0.4) (layer F.Cu) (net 9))
 (segment (start 122.445001 72.915001) (end 123.19 73.66) (width 0.4) (layer F.Cu) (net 10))
 (segment (start 122.445001 68.58) (end 122.445001 72.915001) (width 0.4) (layer F.Cu) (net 10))
 (segment (start 123.19 73.66) (end 123.19 93.345) (width 0.4) (layer F.Cu) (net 10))
 (segment (start 122.445001 94.089999) (end 122.445001 98.425) (width 0.4) (layer F.Cu) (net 10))
 (segment (start 123.19 93.345) (end 122.445001 94.089999) (width 0.4) (layer F.Cu) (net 10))
 (segment (start 122.445001 98.425) (end 122.445001 100.439999) (width 0.4) (layer F.Cu) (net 10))
 (segment (start 119.250509 95.960508) (end 119.675001 96.385) (width 0.4) (layer F.Cu) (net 26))
 (segment (start 119.675001 96.385) (end 119.675001 98.425) (width 0.4) (layer F.Cu) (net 26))
 (segment (start 119.675001 70.62) (end 119.250509 71.044492) (width 0.4) (layer F.Cu) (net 26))
 (segment (start 119.250509 71.044492) (end 119.250509 95.960508) (width 0.4) (layer F.Cu) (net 26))
 (segment (start 119.675001 68.58) (end 119.675001 70.62) (width 0.4) (layer F.Cu) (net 26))
 (segment (start 119.675001 98.425) (end 119.675001 100.415999) (width 0.4) (layer F.Cu) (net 26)))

